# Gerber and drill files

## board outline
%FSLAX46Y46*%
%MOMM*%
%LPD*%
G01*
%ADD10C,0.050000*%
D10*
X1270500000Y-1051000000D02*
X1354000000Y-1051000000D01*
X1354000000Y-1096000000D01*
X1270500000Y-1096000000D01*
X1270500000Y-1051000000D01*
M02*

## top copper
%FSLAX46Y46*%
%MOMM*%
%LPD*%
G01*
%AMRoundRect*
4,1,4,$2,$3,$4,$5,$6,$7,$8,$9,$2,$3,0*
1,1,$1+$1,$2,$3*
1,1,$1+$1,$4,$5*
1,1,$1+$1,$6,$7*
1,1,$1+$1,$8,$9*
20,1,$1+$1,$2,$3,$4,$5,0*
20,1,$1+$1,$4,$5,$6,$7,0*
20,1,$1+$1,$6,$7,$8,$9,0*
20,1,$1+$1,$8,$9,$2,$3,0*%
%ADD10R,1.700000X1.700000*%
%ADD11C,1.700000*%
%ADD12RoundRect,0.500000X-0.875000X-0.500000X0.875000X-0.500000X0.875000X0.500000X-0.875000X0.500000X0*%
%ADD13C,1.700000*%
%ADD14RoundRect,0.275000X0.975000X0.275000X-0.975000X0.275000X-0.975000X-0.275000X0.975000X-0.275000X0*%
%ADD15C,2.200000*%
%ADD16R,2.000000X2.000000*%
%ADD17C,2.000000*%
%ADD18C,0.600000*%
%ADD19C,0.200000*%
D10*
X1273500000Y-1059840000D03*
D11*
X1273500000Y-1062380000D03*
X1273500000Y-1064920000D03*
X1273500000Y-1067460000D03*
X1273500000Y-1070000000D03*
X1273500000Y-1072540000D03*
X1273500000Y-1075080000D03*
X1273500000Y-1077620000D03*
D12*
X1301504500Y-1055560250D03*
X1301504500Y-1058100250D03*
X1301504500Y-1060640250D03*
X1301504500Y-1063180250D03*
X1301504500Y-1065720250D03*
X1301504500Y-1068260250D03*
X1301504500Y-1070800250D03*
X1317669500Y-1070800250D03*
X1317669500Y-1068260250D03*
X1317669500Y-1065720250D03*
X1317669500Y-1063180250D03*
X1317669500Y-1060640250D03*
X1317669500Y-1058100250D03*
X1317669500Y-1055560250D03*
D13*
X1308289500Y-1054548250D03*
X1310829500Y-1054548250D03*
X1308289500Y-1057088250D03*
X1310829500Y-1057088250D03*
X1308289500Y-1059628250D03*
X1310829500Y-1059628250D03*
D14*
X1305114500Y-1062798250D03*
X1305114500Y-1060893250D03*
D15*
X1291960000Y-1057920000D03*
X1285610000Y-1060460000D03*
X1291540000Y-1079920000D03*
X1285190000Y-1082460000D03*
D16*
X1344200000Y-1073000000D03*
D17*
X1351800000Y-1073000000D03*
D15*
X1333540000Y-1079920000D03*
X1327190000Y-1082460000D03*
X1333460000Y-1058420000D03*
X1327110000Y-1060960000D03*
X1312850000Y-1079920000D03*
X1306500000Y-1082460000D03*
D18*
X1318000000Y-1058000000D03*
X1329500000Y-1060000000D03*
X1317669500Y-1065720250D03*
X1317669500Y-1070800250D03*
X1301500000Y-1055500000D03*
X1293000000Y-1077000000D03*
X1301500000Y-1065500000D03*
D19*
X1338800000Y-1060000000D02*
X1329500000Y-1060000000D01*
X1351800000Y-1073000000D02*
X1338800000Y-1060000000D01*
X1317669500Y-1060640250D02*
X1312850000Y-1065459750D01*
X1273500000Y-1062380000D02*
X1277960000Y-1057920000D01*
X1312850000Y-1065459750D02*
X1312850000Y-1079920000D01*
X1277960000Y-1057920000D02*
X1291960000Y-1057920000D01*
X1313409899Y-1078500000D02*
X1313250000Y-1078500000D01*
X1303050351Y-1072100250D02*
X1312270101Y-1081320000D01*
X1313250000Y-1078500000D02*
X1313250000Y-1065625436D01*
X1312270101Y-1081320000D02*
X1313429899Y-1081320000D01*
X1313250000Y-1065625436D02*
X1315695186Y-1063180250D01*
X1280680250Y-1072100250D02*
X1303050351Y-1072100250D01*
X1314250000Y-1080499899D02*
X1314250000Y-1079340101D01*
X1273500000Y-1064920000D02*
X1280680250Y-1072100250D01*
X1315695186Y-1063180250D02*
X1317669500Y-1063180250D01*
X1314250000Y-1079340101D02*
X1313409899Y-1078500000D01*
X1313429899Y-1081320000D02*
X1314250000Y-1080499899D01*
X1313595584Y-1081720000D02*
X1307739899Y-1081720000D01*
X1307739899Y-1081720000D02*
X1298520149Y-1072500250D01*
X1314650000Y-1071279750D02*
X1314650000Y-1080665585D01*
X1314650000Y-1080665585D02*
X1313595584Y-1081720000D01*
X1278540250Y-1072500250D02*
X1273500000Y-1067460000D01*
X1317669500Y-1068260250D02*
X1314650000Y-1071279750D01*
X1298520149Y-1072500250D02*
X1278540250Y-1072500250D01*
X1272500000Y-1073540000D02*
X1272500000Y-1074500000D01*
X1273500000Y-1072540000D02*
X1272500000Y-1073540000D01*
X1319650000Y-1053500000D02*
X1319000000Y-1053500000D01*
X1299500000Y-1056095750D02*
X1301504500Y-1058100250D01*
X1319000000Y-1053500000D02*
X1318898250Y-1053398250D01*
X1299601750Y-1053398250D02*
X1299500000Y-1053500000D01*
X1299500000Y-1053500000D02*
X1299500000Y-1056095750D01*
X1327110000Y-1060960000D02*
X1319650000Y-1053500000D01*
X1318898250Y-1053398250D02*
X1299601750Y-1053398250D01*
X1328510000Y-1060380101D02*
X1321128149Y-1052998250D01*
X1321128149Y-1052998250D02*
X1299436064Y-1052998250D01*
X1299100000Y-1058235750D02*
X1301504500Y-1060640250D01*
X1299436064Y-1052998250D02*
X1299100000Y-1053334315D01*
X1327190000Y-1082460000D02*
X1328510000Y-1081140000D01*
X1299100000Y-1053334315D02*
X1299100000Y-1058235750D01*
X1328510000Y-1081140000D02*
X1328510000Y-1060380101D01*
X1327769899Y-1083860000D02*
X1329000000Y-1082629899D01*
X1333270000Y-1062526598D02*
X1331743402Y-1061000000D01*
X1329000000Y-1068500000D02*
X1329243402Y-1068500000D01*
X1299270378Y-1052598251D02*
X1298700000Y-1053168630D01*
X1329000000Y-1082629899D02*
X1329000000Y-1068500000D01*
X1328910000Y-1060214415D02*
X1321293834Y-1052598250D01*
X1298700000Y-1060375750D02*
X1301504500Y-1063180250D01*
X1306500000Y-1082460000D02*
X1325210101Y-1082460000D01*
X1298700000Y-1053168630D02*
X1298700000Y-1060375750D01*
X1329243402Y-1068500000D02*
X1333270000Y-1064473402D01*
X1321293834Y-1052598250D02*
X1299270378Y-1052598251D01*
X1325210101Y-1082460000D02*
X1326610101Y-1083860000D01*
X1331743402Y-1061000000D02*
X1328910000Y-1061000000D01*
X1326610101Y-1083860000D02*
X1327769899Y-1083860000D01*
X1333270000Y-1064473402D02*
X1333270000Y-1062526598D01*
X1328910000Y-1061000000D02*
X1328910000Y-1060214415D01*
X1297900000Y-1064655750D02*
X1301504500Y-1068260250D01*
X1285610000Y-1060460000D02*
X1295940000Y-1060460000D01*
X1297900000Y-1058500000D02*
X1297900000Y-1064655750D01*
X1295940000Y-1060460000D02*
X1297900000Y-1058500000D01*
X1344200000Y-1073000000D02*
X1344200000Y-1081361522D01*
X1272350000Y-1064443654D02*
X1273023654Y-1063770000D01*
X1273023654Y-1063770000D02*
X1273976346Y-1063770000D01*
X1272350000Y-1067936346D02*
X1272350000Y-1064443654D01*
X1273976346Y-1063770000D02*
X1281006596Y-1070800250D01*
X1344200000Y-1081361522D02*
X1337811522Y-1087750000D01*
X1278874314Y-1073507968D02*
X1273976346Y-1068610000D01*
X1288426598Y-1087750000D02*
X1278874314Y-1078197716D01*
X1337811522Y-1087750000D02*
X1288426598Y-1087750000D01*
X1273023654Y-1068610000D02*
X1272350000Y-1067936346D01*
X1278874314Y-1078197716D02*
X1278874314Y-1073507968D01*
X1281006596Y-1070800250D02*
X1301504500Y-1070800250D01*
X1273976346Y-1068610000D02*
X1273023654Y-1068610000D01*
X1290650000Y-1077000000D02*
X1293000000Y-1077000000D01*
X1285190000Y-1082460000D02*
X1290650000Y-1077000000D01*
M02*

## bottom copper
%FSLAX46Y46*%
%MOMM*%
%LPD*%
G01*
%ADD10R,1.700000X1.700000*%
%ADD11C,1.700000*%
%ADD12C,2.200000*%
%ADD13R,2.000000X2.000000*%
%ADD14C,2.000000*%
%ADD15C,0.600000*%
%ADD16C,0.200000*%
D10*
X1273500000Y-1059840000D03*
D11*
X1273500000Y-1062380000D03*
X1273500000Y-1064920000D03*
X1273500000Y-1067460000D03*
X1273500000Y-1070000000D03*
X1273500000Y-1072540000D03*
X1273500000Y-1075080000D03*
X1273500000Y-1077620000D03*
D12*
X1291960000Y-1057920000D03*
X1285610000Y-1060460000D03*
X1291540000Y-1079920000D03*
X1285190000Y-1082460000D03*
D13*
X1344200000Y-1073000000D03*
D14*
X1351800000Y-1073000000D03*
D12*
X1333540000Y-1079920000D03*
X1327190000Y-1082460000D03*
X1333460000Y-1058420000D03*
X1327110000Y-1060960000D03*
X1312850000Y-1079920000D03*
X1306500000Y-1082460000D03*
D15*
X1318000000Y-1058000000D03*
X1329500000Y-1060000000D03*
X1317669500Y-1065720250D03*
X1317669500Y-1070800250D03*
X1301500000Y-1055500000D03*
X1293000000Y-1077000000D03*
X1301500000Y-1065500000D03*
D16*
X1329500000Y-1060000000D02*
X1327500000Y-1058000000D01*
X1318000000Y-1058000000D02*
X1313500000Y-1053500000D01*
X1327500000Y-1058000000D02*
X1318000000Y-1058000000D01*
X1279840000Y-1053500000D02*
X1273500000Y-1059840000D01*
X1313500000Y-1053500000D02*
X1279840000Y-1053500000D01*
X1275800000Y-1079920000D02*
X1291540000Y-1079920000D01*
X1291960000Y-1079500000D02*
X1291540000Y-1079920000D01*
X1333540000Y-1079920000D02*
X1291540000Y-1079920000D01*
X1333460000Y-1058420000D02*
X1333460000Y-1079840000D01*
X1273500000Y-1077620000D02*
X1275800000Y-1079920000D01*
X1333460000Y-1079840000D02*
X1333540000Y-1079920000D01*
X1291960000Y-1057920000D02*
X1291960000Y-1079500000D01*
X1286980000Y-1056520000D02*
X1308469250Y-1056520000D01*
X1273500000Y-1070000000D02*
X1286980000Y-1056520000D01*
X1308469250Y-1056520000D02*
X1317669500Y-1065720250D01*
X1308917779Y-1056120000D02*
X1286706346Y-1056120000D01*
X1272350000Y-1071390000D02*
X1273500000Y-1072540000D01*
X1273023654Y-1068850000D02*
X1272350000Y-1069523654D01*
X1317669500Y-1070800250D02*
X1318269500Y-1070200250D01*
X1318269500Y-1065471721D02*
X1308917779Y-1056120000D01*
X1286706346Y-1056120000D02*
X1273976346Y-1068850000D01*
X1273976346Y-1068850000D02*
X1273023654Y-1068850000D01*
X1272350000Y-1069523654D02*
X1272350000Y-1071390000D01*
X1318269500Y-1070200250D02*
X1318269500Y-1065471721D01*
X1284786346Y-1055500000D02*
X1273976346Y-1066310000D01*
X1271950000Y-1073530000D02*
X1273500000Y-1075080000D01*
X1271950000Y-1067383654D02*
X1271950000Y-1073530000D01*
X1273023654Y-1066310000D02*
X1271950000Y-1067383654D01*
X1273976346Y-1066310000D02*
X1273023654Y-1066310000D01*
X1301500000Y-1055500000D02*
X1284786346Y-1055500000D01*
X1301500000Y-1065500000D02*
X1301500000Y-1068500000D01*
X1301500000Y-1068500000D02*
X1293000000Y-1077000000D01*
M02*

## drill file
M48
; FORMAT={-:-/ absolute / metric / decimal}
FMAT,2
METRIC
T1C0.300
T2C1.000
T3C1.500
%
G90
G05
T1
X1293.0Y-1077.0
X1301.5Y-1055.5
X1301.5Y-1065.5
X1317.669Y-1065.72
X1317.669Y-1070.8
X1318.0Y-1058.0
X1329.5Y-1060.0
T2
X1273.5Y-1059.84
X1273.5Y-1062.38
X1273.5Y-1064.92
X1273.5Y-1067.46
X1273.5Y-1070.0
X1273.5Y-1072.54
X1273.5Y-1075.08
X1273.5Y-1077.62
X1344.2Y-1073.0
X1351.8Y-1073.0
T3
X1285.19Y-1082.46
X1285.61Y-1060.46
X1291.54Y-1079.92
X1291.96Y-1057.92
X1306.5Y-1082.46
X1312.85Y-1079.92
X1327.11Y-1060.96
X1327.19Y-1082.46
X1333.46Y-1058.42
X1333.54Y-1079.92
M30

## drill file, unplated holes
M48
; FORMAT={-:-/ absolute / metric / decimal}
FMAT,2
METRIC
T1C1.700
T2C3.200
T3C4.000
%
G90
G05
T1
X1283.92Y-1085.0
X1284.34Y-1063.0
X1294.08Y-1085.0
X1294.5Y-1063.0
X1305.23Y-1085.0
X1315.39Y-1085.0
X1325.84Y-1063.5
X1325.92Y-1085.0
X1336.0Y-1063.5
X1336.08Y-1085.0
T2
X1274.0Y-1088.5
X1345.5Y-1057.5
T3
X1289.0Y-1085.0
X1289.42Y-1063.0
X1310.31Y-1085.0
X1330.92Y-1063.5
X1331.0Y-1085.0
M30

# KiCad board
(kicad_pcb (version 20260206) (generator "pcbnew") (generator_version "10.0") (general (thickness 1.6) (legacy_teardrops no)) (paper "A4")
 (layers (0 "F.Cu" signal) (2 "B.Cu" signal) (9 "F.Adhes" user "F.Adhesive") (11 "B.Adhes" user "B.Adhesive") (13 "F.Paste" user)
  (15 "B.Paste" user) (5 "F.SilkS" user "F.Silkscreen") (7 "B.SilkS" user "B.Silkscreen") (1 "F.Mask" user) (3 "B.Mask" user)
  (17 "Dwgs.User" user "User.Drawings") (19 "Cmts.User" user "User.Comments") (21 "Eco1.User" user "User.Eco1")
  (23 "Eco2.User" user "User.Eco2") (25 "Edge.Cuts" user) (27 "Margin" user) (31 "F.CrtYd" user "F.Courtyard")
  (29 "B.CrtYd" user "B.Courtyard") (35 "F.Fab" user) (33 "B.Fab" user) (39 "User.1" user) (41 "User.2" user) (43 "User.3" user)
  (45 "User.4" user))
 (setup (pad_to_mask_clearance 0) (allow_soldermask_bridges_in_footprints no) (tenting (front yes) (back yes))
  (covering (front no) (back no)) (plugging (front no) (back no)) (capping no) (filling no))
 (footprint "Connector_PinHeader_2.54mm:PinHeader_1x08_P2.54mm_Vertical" (layer "F.Cu") (at 1273.5 1059.84)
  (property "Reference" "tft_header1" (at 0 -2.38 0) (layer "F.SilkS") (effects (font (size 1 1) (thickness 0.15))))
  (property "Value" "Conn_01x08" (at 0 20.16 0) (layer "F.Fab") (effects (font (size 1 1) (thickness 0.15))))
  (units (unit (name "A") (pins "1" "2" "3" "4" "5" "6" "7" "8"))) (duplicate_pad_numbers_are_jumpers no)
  (pad "1" thru_hole rect (at 0 0) (size 1.7 1.7) (drill 1) (layers "*.Cu" "*.Mask") (remove_unused_layers no) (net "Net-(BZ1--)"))
  (pad "2" thru_hole circle (at 0 2.54) (size 1.7 1.7) (drill 1) (layers "*.Cu" "*.Mask") (remove_unused_layers no) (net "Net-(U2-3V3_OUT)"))
  (pad "3" thru_hole circle (at 0 5.08) (size 1.7 1.7) (drill 1) (layers "*.Cu" "*.Mask") (remove_unused_layers no) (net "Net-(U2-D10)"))
  (pad "4" thru_hole circle (at 0 7.62) (size 1.7 1.7) (drill 1) (layers "*.Cu" "*.Mask") (remove_unused_layers no) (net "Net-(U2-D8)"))
  (pad "5" thru_hole circle (at 0 10.16) (size 1.7 1.7) (drill 1) (layers "*.Cu" "*.Mask") (remove_unused_layers no)
   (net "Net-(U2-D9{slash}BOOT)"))
  (pad "6" thru_hole circle (at 0 12.7) (size 1.7 1.7) (drill 1) (layers "*.Cu" "*.Mask") (remove_unused_layers no) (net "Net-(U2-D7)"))
  (pad "7" thru_hole circle (at 0 15.24) (size 1.7 1.7) (drill 1) (layers "*.Cu" "*.Mask") (remove_unused_layers no) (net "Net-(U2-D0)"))
  (pad "8" thru_hole circle (at 0 17.78) (size 1.7 1.7) (drill 1) (layers "*.Cu" "*.Mask") (remove_unused_layers no)
   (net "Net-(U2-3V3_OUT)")))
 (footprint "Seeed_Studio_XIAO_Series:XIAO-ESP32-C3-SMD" (layer "F.Cu") (at 1300.6695 1073.68025)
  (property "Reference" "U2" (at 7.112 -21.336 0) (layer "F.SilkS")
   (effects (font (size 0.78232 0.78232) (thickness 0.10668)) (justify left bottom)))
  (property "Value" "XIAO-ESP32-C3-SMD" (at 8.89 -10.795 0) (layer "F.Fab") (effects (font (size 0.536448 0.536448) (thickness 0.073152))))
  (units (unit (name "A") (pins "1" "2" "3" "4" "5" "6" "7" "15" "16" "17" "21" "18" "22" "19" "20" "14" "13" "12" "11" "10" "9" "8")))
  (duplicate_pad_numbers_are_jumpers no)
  (pad "1" smd roundrect (at 0.835 -18.12) (size 2.75 2) (layers "F.Cu" "F.Mask" "F.Paste") (roundrect_rratio 0.25) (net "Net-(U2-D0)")
   (solder_mask_margin 0.0508) (thermal_bridge_angle 45))
  (pad "2" smd roundrect (at 0.835 -15.58) (size 2.75 2) (layers "F.Cu" "F.Mask" "F.Paste") (roundrect_rratio 0.25) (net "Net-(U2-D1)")
   (solder_mask_margin 0.0508) (thermal_bridge_angle 45))
  (pad "3" smd roundrect (at 0.835 -13.04) (size 2.75 2) (layers "F.Cu" "F.Mask" "F.Paste") (roundrect_rratio 0.25) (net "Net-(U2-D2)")
   (solder_mask_margin 0.0508) (thermal_bridge_angle 45))
  (pad "4" smd roundrect (at 0.835 -10.5) (size 2.75 2) (layers "F.Cu" "F.Mask" "F.Paste") (roundrect_rratio 0.25) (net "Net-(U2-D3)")
   (solder_mask_margin 0.0508) (thermal_bridge_angle 45))
  (pad "5" smd roundrect (at 0.835 -7.96) (size 2.75 2) (layers "F.Cu" "F.Mask" "F.Paste") (roundrect_rratio 0.25) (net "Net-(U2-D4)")
   (solder_mask_margin 0.0508) (thermal_bridge_angle 45))
  (pad "6" smd roundrect (at 0.835 -5.42) (size 2.75 2) (layers "F.Cu" "F.Mask" "F.Paste") (roundrect_rratio 0.25) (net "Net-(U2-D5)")
   (solder_mask_margin 0.0508) (thermal_bridge_angle 45))
  (pad "7" smd roundrect (at 0.835 -2.88) (size 2.75 2) (layers "F.Cu" "F.Mask" "F.Paste") (roundrect_rratio 0.25) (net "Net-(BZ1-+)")
   (solder_mask_margin 0.0508) (thermal_bridge_angle 45))
  (pad "8" smd roundrect (at 17 -2.88) (size 2.75 2) (layers "F.Cu" "F.Mask" "F.Paste") (roundrect_rratio 0.25) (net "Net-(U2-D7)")
   (solder_mask_margin 0.0508) (thermal_bridge_angle 45))
  (pad "9" smd roundrect (at 17 -5.42) (size 2.75 2) (layers "F.Cu" "F.Mask" "F.Paste") (roundrect_rratio 0.25) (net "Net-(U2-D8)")
   (solder_mask_margin 0.0508) (thermal_bridge_angle 45))
  (pad "10" smd roundrect (at 17 -7.96) (size 2.75 2) (layers "F.Cu" "F.Mask" "F.Paste") (roundrect_rratio 0.25)
   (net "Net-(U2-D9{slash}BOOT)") (solder_mask_margin 0.0508) (thermal_bridge_angle 45))
  (pad "11" smd roundrect (at 17 -10.5) (size 2.75 2) (layers "F.Cu" "F.Mask" "F.Paste") (roundrect_rratio 0.25) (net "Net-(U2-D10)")
   (solder_mask_margin 0.0508) (thermal_bridge_angle 45))
  (pad "12" smd roundrect (at 17 -13.04) (size 2.75 2) (layers "F.Cu" "F.Mask" "F.Paste") (roundrect_rratio 0.25) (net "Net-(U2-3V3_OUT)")
   (solder_mask_margin 0.0508) (thermal_bridge_angle 45))
  (pad "13" smd roundrect (at 17 -15.58) (size 2.75 2) (layers "F.Cu" "F.Mask" "F.Paste") (roundrect_rratio 0.25) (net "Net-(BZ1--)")
   (solder_mask_margin 0.0508) (thermal_bridge_angle 45))
  (pad "14" smd roundrect (at 17 -18.12) (size 2.75 2) (layers "F.Cu" "F.Mask" "F.Paste") (roundrect_rratio 0.25)
   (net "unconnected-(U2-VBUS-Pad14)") (solder_mask_margin 0.0508) (thermal_bridge_angle 45))
  (pad "15" smd circle (at 7.62 -19.132) (size 1.7 1.7) (layers "F.Cu" "F.Mask" "F.Paste") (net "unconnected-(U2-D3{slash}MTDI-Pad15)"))
  (pad "16" smd circle (at 10.16 -19.132) (size 1.7 1.7) (layers "F.Cu" "F.Mask" "F.Paste") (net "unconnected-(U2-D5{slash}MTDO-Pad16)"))
  (pad "17" smd circle (at 7.62 -16.592) (size 1.7 1.7) (layers "F.Cu" "F.Mask" "F.Paste") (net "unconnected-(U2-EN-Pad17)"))
  (pad "18" smd circle (at 10.16 -16.592) (size 1.7 1.7) (layers "F.Cu" "F.Mask" "F.Paste") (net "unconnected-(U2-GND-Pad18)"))
  (pad "19" smd circle (at 7.62 -14.052) (size 1.7 1.7) (layers "F.Cu" "F.Mask" "F.Paste") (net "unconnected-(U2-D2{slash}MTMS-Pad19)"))
  (pad "20" smd circle (at 10.16 -14.052) (size 1.7 1.7) (layers "F.Cu" "F.Mask" "F.Paste") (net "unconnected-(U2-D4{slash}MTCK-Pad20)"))
  (pad "21" smd roundrect (at 4.445 -10.882 180) (size 2.5 1.1) (layers "F.Cu" "F.Mask" "F.Paste") (roundrect_rratio 0.25)
   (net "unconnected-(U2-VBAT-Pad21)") (thermal_bridge_angle 45))
  (pad "22" smd roundrect (at 4.445 -12.787 180) (size 2.5 1.1) (layers "F.Cu" "F.Mask" "F.Paste") (roundrect_rratio 0.25)
   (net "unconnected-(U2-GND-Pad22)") (thermal_bridge_angle 45)))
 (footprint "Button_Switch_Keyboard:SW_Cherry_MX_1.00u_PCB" (layer "F.Cu") (at 1291.96 1057.92)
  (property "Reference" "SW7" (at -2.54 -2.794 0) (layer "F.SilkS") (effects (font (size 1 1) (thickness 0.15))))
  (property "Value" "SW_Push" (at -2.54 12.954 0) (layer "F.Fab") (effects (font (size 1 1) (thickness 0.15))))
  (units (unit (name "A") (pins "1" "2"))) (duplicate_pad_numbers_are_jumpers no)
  (pad "" np_thru_hole circle (at -7.62 5.08) (size 1.7 1.7) (drill 1.7) (layers "*.Cu" "*.Mask"))
  (pad "" np_thru_hole circle (at -2.54 5.08) (size 4 4) (drill 4) (layers "*.Cu" "*.Mask"))
  (pad "" np_thru_hole circle (at 2.54 5.08) (size 1.7 1.7) (drill 1.7) (layers "*.Cu" "*.Mask"))
  (pad "1" thru_hole circle (at 0 0) (size 2.2 2.2) (drill 1.5) (layers "*.Cu" "*.Mask") (remove_unused_layers no) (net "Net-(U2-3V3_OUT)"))
  (pad "2" thru_hole circle (at -6.35 2.54) (size 2.2 2.2) (drill 1.5) (layers "*.Cu" "*.Mask") (remove_unused_layers no)
   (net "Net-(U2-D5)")))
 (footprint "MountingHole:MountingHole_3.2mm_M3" (layer "F.Cu") (at 1345.5 1057.5)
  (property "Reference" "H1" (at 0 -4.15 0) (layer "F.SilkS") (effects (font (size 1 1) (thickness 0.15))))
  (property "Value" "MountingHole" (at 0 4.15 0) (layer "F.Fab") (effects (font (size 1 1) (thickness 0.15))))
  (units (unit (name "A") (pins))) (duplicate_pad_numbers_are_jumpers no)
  (pad "" np_thru_hole circle (at 0 0) (size 3.2 3.2) (drill 3.2) (layers "*.Cu" "*.Mask")))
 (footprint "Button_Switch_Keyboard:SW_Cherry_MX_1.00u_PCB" (layer "F.Cu") (at 1291.54 1079.92)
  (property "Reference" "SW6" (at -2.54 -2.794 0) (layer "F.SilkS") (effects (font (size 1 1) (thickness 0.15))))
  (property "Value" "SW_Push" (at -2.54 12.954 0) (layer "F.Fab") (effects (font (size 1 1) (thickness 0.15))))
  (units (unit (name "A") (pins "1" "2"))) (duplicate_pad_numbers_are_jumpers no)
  (pad "" np_thru_hole circle (at -7.62 5.08) (size 1.7 1.7) (drill 1.7) (layers "*.Cu" "*.Mask"))
  (pad "" np_thru_hole circle (at -2.54 5.08) (size 4 4) (drill 4) (layers "*.Cu" "*.Mask"))
  (pad "" np_thru_hole circle (at 2.54 5.08) (size 1.7 1.7) (drill 1.7) (layers "*.Cu" "*.Mask"))
  (pad "1" thru_hole circle (at 0 0) (size 2.2 2.2) (drill 1.5) (layers "*.Cu" "*.Mask") (remove_unused_layers no) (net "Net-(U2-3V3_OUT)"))
  (pad "2" thru_hole circle (at -6.35 2.54) (size 2.2 2.2) (drill 1.5) (layers "*.Cu" "*.Mask") (remove_unused_layers no)
   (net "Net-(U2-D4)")))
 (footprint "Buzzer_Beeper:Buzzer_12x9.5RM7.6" (layer "F.Cu") (at 1344.2 1073)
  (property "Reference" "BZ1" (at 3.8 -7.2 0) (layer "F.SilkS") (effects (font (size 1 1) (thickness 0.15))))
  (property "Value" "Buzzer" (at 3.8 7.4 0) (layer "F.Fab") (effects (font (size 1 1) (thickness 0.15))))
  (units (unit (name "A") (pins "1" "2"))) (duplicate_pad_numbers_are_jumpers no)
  (pad "1" thru_hole rect (at 0 0) (size 2 2) (drill 1) (layers "*.Cu" "*.Mask") (remove_unused_layers no) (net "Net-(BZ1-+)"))
  (pad "2" thru_hole circle (at 7.6 0) (size 2 2) (drill 1) (layers "*.Cu" "*.Mask") (remove_unused_layers no) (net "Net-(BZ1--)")))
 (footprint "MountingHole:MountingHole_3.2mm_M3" (layer "F.Cu") (at 1274 1088.5)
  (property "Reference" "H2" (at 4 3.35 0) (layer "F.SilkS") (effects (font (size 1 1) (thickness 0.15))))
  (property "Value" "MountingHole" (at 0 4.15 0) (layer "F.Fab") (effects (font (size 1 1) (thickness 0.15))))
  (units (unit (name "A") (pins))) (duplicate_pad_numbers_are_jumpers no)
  (pad "" np_thru_hole circle (at 0 0) (size 3.2 3.2) (drill 3.2) (layers "*.Cu" "*.Mask")))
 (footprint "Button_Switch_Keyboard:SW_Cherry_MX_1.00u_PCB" (layer "F.Cu") (at 1333.54 1079.92)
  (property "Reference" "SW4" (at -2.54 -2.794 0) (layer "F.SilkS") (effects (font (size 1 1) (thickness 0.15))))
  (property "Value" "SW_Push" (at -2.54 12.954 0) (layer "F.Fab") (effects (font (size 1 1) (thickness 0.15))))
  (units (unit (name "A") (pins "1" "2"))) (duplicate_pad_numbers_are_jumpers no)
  (pad "" np_thru_hole circle (at -7.62 5.08) (size 1.7 1.7) (drill 1.7) (layers "*.Cu" "*.Mask"))
  (pad "" np_thru_hole circle (at -2.54 5.08) (size 4 4) (drill 4) (layers "*.Cu" "*.Mask"))
  (pad "" np_thru_hole circle (at 2.54 5.08) (size 1.7 1.7) (drill 1.7) (layers "*.Cu" "*.Mask"))
  (pad "1" thru_hole circle (at 0 0) (size 2.2 2.2) (drill 1.5) (layers "*.Cu" "*.Mask") (remove_unused_layers no) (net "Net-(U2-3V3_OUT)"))
  (pad "2" thru_hole circle (at -6.35 2.54) (size 2.2 2.2) (drill 1.5) (layers "*.Cu" "*.Mask") (remove_unused_layers no)
   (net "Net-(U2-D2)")))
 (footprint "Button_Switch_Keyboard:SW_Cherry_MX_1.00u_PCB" (layer "F.Cu") (at 1333.46 1058.42)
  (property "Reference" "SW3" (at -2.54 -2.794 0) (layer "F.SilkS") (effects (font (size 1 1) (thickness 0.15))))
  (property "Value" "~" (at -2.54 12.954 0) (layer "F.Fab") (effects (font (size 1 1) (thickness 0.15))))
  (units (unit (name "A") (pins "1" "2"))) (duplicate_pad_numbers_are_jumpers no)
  (pad "" np_thru_hole circle (at -7.62 5.08) (size 1.7 1.7) (drill 1.7) (layers "*.Cu" "*.Mask"))
  (pad "" np_thru_hole circle (at -2.54 5.08) (size 4 4) (drill 4) (layers "*.Cu" "*.Mask"))
  (pad "" np_thru_hole circle (at 2.54 5.08) (size 1.7 1.7) (drill 1.7) (layers "*.Cu" "*.Mask"))
  (pad "1" thru_hole circle (at 0 0) (size 2.2 2.2) (drill 1.5) (layers "*.Cu" "*.Mask") (remove_unused_layers no) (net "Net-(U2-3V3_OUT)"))
  (pad "2" thru_hole circle (at -6.35 2.54) (size 2.2 2.2) (drill 1.5) (layers "*.Cu" "*.Mask") (remove_unused_layers no)
   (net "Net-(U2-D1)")))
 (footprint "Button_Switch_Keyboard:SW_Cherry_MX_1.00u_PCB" (layer "F.Cu") (at 1312.85 1079.92)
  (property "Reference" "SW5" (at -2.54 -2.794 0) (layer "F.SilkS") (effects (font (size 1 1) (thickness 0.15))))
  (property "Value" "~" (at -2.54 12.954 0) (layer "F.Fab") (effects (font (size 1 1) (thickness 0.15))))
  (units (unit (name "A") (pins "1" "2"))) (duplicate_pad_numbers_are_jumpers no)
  (pad "" np_thru_hole circle (at -7.62 5.08) (size 1.7 1.7) (drill 1.7) (layers "*.Cu" "*.Mask"))
  (pad "" np_thru_hole circle (at -2.54 5.08) (size 4 4) (drill 4) (layers "*.Cu" "*.Mask"))
  (pad "" np_thru_hole circle (at 2.54 5.08) (size 1.7 1.7) (drill 1.7) (layers "*.Cu" "*.Mask"))
  (pad "1" thru_hole circle (at 0 0) (size 2.2 2.2) (drill 1.5) (layers "*.Cu" "*.Mask") (remove_unused_layers no) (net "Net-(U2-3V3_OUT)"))
  (pad "2" thru_hole circle (at -6.35 2.54) (size 2.2 2.2) (drill 1.5) (layers "*.Cu" "*.Mask") (remove_unused_layers no)
   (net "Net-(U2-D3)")))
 (gr_rect (start 1270.5 1051) (end 1354 1096) (stroke (width 0.05) (type default)) (fill no) (layer "Edge.Cuts"))
 (segment (start 1338.8 1060) (end 1329.5 1060) (width 0.2) (layer "F.Cu") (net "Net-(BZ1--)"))
 (segment (start 1351.8 1073) (end 1338.8 1060) (width 0.2) (layer "F.Cu") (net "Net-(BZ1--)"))
 (via (at 1318 1058) (size 0.6) (drill 0.3) (layers "F.Cu" "B.Cu") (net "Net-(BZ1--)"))
 (via (at 1329.5 1060) (size 0.6) (drill 0.3) (layers "F.Cu" "B.Cu") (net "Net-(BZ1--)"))
 (segment (start 1329.5 1060) (end 1327.5 1058) (width 0.2) (layer "B.Cu") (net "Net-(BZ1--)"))
 (segment (start 1318 1058) (end 1313.5 1053.5) (width 0.2) (layer "B.Cu") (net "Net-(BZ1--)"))
 (segment (start 1327.5 1058) (end 1318 1058) (width 0.2) (layer "B.Cu") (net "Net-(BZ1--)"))
 (segment (start 1279.84 1053.5) (end 1273.5 1059.84) (width 0.2) (layer "B.Cu") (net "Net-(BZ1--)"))
 (segment (start 1313.5 1053.5) (end 1279.84 1053.5) (width 0.2) (layer "B.Cu") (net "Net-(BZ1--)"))
 (segment (start 1317.6695 1060.64025) (end 1312.85 1065.45975) (width 0.2) (layer "F.Cu") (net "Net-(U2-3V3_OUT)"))
 (segment (start 1273.5 1062.38) (end 1277.96 1057.92) (width 0.2) (layer "F.Cu") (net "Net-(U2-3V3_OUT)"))
 (segment (start 1312.85 1065.45975) (end 1312.85 1079.92) (width 0.2) (layer "F.Cu") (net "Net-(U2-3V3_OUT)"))
 (segment (start 1277.96 1057.92) (end 1291.96 1057.92) (width 0.2) (layer "F.Cu") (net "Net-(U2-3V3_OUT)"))
 (segment (start 1275.8 1079.92) (end 1291.54 1079.92) (width 0.2) (layer "B.Cu") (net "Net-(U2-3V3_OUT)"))
 (segment (start 1291.96 1079.5) (end 1291.54 1079.92) (width 0.2) (layer "B.Cu") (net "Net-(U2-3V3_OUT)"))
 (segment (start 1333.54 1079.92) (end 1291.54 1079.92) (width 0.2) (layer "B.Cu") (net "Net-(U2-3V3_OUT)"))
 (segment (start 1333.46 1058.42) (end 1333.46 1079.84) (width 0.2) (layer "B.Cu") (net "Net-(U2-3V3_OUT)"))
 (segment (start 1273.5 1077.62) (end 1275.8 1079.92) (width 0.2) (layer "B.Cu") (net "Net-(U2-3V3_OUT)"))
 (segment (start 1333.46 1079.84) (end 1333.54 1079.92) (width 0.2) (layer "B.Cu") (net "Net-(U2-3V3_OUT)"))
 (segment (start 1291.96 1057.92) (end 1291.96 1079.5) (width 0.2) (layer "B.Cu") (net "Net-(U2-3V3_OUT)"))
 (segment (start 1313.409899 1078.5) (end 1313.25 1078.5) (width 0.2) (layer "F.Cu") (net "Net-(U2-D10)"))
 (segment (start 1303.050351 1072.10025) (end 1312.270101 1081.32) (width 0.2) (layer "F.Cu") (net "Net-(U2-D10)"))
 (segment (start 1313.25 1078.5) (end 1313.25 1065.625436) (width 0.2) (layer "F.Cu") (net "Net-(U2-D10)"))
 (segment (start 1312.270101 1081.32) (end 1313.429899 1081.32) (width 0.2) (layer "F.Cu") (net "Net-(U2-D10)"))
 (segment (start 1313.25 1065.625436) (end 1315.695186 1063.18025) (width 0.2) (layer "F.Cu") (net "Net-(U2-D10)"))
 (segment (start 1280.68025 1072.10025) (end 1303.050351 1072.10025) (width 0.2) (layer "F.Cu") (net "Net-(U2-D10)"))
 (segment (start 1314.25 1080.499899) (end 1314.25 1079.340101) (width 0.2) (layer "F.Cu") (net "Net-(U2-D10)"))
 (segment (start 1273.5 1064.92) (end 1280.68025 1072.10025) (width 0.2) (layer "F.Cu") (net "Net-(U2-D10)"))
 (segment (start 1315.695186 1063.18025) (end 1317.6695 1063.18025) (width 0.2) (layer "F.Cu") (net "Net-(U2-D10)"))
 (segment (start 1314.25 1079.340101) (end 1313.409899 1078.5) (width 0.2) (layer "F.Cu") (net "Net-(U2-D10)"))
 (segment (start 1313.429899 1081.32) (end 1314.25 1080.499899) (width 0.2) (layer "F.Cu") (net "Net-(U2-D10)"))
 (segment (start 1313.595584 1081.72) (end 1307.739899 1081.72) (width 0.2) (layer "F.Cu") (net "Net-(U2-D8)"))
 (segment (start 1307.739899 1081.72) (end 1298.520149 1072.50025) (width 0.2) (layer "F.Cu") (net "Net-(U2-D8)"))
 (segment (start 1314.65 1071.27975) (end 1314.65 1080.665585) (width 0.2) (layer "F.Cu") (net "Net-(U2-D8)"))
 (segment (start 1314.65 1080.665585) (end 1313.595584 1081.72) (width 0.2) (layer "F.Cu") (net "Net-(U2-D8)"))
 (segment (start 1278.54025 1072.50025) (end 1273.5 1067.46) (width 0.2) (layer "F.Cu") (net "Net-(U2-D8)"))
 (segment (start 1317.6695 1068.26025) (end 1314.65 1071.27975) (width 0.2) (layer "F.Cu") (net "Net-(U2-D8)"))
 (segment (start 1298.520149 1072.50025) (end 1278.54025 1072.50025) (width 0.2) (layer "F.Cu") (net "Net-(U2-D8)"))
 (via (at 1317.6695 1065.72025) (size 0.6) (drill 0.3) (layers "F.Cu" "B.Cu") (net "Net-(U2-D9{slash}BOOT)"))
 (segment (start 1286.98 1056.52) (end 1308.46925 1056.52) (width 0.2) (layer "B.Cu") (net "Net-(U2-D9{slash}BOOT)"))
 (segment (start 1273.5 1070) (end 1286.98 1056.52) (width 0.2) (layer "B.Cu") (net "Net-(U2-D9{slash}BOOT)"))
 (segment (start 1308.46925 1056.52) (end 1317.6695 1065.72025) (width 0.2) (layer "B.Cu") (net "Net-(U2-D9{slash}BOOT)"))
 (segment (start 1272.5 1073.54) (end 1272.5 1074.5) (width 0.2) (layer "F.Cu") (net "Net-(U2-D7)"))
 (segment (start 1273.5 1072.54) (end 1272.5 1073.54) (width 0.2) (layer "F.Cu") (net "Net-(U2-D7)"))
 (via (at 1317.6695 1070.80025) (size 0.6) (drill 0.3) (layers "F.Cu" "B.Cu") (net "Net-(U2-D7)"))
 (segment (start 1308.917779 1056.12) (end 1286.706346 1056.12) (width 0.2) (layer "B.Cu") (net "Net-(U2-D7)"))
 (segment (start 1272.35 1071.39) (end 1273.5 1072.54) (width 0.2) (layer "B.Cu") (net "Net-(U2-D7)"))
 (segment (start 1273.023654 1068.85) (end 1272.35 1069.523654) (width 0.2) (layer "B.Cu") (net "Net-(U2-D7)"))
 (segment (start 1317.6695 1070.80025) (end 1318.2695 1070.20025) (width 0.2) (layer "B.Cu") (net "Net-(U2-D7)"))
 (segment (start 1318.2695 1065.471721) (end 1308.917779 1056.12) (width 0.2) (layer "B.Cu") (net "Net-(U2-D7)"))
 (segment (start 1286.706346 1056.12) (end 1273.976346 1068.85) (width 0.2) (layer "B.Cu") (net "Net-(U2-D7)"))
 (segment (start 1273.976346 1068.85) (end 1273.023654 1068.85) (width 0.2) (layer "B.Cu") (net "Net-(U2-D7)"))
 (segment (start 1272.35 1069.523654) (end 1272.35 1071.39) (width 0.2) (layer "B.Cu") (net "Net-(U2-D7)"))
 (segment (start 1318.2695 1070.20025) (end 1318.2695 1065.471721) (width 0.2) (layer "B.Cu") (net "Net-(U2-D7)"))
 (via (at 1301.5 1055.5) (size 0.6) (drill 0.3) (layers "F.Cu" "B.Cu") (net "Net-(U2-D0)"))
 (segment (start 1284.786346 1055.5) (end 1273.976346 1066.31) (width 0.2) (layer "B.Cu") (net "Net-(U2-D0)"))
 (segment (start 1271.95 1073.53) (end 1273.5 1075.08) (width 0.2) (layer "B.Cu") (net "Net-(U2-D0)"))
 (segment (start 1271.95 1067.383654) (end 1271.95 1073.53) (width 0.2) (layer "B.Cu") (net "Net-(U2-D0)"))
 (segment (start 1273.023654 1066.31) (end 1271.95 1067.383654) (width 0.2) (layer "B.Cu") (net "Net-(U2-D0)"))
 (segment (start 1273.976346 1066.31) (end 1273.023654 1066.31) (width 0.2) (layer "B.Cu") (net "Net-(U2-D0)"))
 (segment (start 1301.5 1055.5) (end 1284.786346 1055.5) (width 0.2) (layer "B.Cu") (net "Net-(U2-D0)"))
 (segment (start 1319.65 1053.5) (end 1319 1053.5) (width 0.2) (layer "F.Cu") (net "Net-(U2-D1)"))
 (segment (start 1299.5 1056.09575) (end 1301.5045 1058.10025) (width 0.2) (layer "F.Cu") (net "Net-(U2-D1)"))
 (segment (start 1319 1053.5) (end 1318.89825 1053.39825) (width 0.2) (layer "F.Cu") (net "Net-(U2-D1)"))
 (segment (start 1299.60175 1053.39825) (end 1299.5 1053.5) (width 0.2) (layer "F.Cu") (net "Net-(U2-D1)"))
 (segment (start 1299.5 1053.5) (end 1299.5 1056.09575) (width 0.2) (layer "F.Cu") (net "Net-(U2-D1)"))
 (segment (start 1327.11 1060.96) (end 1319.65 1053.5) (width 0.2) (layer "F.Cu") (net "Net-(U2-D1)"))
 (segment (start 1318.89825 1053.39825) (end 1299.60175 1053.39825) (width 0.2) (layer "F.Cu") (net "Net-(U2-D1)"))
 (segment (start 1328.51 1060.380101) (end 1321.128149 1052.99825) (width 0.2) (layer "F.Cu") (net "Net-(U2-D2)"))
 (segment (start 1321.128149 1052.99825) (end 1299.436064 1052.99825) (width 0.2) (layer "F.Cu") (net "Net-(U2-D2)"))
 (segment (start 1299.1 1058.23575) (end 1301.5045 1060.64025) (width 0.2) (layer "F.Cu") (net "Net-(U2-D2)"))
 (segment (start 1299.436064 1052.99825) (end 1299.1 1053.334315) (width 0.2) (layer "F.Cu") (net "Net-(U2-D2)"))
 (segment (start 1327.19 1082.46) (end 1328.51 1081.14) (width 0.2) (layer "F.Cu") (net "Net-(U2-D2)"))
 (segment (start 1299.1 1053.334315) (end 1299.1 1058.23575) (width 0.2) (layer "F.Cu") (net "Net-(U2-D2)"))
 (segment (start 1328.51 1081.14) (end 1328.51 1060.380101) (width 0.2) (layer "F.Cu") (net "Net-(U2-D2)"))
 (segment (start 1327.769899 1083.86) (end 1329 1082.629899) (width 0.2) (layer "F.Cu") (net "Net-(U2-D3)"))
 (segment (start 1333.27 1062.526598) (end 1331.743402 1061) (width 0.2) (layer "F.Cu") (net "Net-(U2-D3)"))
 (segment (start 1329 1068.5) (end 1329.243402 1068.5) (width 0.2) (layer "F.Cu") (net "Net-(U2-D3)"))
 (segment (start 1299.270378 1052.598251) (end 1298.7 1053.16863) (width 0.2) (layer "F.Cu") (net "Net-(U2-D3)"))
 (segment (start 1329 1082.629899) (end 1329 1068.5) (width 0.2) (layer "F.Cu") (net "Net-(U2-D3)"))
 (segment (start 1328.91 1060.214415) (end 1321.293834 1052.59825) (width 0.2) (layer "F.Cu") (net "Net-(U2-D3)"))
 (segment (start 1298.7 1060.37575) (end 1301.5045 1063.18025) (width 0.2) (layer "F.Cu") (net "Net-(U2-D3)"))
 (segment (start 1306.5 1082.46) (end 1325.210101 1082.46) (width 0.2) (layer "F.Cu") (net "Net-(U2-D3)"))
 (segment (start 1298.7 1053.16863) (end 1298.7 1060.37575) (width 0.2) (layer "F.Cu") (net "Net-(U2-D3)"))
 (segment (start 1329.243402 1068.5) (end 1333.27 1064.473402) (width 0.2) (layer "F.Cu") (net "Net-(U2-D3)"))
 (segment (start 1321.293834 1052.59825) (end 1299.270378 1052.598251) (width 0.2) (layer "F.Cu") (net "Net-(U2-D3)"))
 (segment (start 1325.210101 1082.46) (end 1326.610101 1083.86) (width 0.2) (layer "F.Cu") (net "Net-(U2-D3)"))
 (segment (start 1331.743402 1061) (end 1328.91 1061) (width 0.2) (layer "F.Cu") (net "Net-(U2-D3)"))
 (segment (start 1326.610101 1083.86) (end 1327.769899 1083.86) (width 0.2) (layer "F.Cu") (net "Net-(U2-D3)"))
 (segment (start 1333.27 1064.473402) (end 1333.27 1062.526598) (width 0.2) (layer "F.Cu") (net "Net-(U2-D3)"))
 (segment (start 1328.91 1061) (end 1328.91 1060.214415) (width 0.2) (layer "F.Cu") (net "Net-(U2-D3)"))
 (segment (start 1297.9 1064.65575) (end 1301.5045 1068.26025) (width 0.2) (layer "F.Cu") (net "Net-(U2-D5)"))
 (segment (start 1285.61 1060.46) (end 1295.94 1060.46) (width 0.2) (layer "F.Cu") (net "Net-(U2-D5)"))
 (segment (start 1297.9 1058.5) (end 1297.9 1064.65575) (width 0.2) (layer "F.Cu") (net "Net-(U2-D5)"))
 (segment (start 1295.94 1060.46) (end 1297.9 1058.5) (width 0.2) (layer "F.Cu") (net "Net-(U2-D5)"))
 (segment (start 1344.2 1073) (end 1344.2 1081.361522) (width 0.2) (layer "F.Cu") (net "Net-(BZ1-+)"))
 (segment (start 1272.35 1064.443654) (end 1273.023654 1063.77) (width 0.2) (layer "F.Cu") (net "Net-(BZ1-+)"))
 (segment (start 1273.023654 1063.77) (end 1273.976346 1063.77) (width 0.2) (layer "F.Cu") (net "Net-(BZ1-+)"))
 (segment (start 1272.35 1067.936346) (end 1272.35 1064.443654) (width 0.2) (layer "F.Cu") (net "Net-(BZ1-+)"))
 (segment (start 1273.976346 1063.77) (end 1281.006596 1070.80025) (width 0.2) (layer "F.Cu") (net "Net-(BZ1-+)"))
 (segment (start 1344.2 1081.361522) (end 1337.811522 1087.75) (width 0.2) (layer "F.Cu") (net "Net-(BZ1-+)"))
 (segment (start 1278.874314 1073.507968) (end 1273.976346 1068.61) (width 0.2) (layer "F.Cu") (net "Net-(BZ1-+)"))
 (segment (start 1288.426598 1087.75) (end 1278.874314 1078.197716) (width 0.2) (layer "F.Cu") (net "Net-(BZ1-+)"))
 (segment (start 1337.811522 1087.75) (end 1288.426598 1087.75) (width 0.2) (layer "F.Cu") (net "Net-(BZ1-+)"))
 (segment (start 1273.023654 1068.61) (end 1272.35 1067.936346) (width 0.2) (layer "F.Cu") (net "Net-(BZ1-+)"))
 (segment (start 1278.874314 1078.197716) (end 1278.874314 1073.507968) (width 0.2) (layer "F.Cu") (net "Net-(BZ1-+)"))
 (segment (start 1281.006596 1070.80025) (end 1301.5045 1070.80025) (width 0.2) (layer "F.Cu") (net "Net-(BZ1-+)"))
 (segment (start 1273.976346 1068.61) (end 1273.023654 1068.61) (width 0.2) (layer "F.Cu") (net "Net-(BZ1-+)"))
 (segment (start 1290.65 1077) (end 1293 1077) (width 0.2) (layer "F.Cu") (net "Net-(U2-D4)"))
 (segment (start 1285.19 1082.46) (end 1290.65 1077) (width 0.2) (layer "F.Cu") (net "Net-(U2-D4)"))
 (via (at 1293 1077) (size 0.6) (drill 0.3) (layers "F.Cu" "B.Cu") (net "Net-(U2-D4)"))
 (via (at 1301.5 1065.5) (size 0.6) (drill 0.3) (layers "F.Cu" "B.Cu") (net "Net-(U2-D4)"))
 (segment (start 1301.5 1065.5) (end 1301.5 1068.5) (width 0.2) (layer "B.Cu") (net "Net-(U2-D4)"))
 (segment (start 1301.5 1068.5) (end 1293 1077) (width 0.2) (layer "B.Cu") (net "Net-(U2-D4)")))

